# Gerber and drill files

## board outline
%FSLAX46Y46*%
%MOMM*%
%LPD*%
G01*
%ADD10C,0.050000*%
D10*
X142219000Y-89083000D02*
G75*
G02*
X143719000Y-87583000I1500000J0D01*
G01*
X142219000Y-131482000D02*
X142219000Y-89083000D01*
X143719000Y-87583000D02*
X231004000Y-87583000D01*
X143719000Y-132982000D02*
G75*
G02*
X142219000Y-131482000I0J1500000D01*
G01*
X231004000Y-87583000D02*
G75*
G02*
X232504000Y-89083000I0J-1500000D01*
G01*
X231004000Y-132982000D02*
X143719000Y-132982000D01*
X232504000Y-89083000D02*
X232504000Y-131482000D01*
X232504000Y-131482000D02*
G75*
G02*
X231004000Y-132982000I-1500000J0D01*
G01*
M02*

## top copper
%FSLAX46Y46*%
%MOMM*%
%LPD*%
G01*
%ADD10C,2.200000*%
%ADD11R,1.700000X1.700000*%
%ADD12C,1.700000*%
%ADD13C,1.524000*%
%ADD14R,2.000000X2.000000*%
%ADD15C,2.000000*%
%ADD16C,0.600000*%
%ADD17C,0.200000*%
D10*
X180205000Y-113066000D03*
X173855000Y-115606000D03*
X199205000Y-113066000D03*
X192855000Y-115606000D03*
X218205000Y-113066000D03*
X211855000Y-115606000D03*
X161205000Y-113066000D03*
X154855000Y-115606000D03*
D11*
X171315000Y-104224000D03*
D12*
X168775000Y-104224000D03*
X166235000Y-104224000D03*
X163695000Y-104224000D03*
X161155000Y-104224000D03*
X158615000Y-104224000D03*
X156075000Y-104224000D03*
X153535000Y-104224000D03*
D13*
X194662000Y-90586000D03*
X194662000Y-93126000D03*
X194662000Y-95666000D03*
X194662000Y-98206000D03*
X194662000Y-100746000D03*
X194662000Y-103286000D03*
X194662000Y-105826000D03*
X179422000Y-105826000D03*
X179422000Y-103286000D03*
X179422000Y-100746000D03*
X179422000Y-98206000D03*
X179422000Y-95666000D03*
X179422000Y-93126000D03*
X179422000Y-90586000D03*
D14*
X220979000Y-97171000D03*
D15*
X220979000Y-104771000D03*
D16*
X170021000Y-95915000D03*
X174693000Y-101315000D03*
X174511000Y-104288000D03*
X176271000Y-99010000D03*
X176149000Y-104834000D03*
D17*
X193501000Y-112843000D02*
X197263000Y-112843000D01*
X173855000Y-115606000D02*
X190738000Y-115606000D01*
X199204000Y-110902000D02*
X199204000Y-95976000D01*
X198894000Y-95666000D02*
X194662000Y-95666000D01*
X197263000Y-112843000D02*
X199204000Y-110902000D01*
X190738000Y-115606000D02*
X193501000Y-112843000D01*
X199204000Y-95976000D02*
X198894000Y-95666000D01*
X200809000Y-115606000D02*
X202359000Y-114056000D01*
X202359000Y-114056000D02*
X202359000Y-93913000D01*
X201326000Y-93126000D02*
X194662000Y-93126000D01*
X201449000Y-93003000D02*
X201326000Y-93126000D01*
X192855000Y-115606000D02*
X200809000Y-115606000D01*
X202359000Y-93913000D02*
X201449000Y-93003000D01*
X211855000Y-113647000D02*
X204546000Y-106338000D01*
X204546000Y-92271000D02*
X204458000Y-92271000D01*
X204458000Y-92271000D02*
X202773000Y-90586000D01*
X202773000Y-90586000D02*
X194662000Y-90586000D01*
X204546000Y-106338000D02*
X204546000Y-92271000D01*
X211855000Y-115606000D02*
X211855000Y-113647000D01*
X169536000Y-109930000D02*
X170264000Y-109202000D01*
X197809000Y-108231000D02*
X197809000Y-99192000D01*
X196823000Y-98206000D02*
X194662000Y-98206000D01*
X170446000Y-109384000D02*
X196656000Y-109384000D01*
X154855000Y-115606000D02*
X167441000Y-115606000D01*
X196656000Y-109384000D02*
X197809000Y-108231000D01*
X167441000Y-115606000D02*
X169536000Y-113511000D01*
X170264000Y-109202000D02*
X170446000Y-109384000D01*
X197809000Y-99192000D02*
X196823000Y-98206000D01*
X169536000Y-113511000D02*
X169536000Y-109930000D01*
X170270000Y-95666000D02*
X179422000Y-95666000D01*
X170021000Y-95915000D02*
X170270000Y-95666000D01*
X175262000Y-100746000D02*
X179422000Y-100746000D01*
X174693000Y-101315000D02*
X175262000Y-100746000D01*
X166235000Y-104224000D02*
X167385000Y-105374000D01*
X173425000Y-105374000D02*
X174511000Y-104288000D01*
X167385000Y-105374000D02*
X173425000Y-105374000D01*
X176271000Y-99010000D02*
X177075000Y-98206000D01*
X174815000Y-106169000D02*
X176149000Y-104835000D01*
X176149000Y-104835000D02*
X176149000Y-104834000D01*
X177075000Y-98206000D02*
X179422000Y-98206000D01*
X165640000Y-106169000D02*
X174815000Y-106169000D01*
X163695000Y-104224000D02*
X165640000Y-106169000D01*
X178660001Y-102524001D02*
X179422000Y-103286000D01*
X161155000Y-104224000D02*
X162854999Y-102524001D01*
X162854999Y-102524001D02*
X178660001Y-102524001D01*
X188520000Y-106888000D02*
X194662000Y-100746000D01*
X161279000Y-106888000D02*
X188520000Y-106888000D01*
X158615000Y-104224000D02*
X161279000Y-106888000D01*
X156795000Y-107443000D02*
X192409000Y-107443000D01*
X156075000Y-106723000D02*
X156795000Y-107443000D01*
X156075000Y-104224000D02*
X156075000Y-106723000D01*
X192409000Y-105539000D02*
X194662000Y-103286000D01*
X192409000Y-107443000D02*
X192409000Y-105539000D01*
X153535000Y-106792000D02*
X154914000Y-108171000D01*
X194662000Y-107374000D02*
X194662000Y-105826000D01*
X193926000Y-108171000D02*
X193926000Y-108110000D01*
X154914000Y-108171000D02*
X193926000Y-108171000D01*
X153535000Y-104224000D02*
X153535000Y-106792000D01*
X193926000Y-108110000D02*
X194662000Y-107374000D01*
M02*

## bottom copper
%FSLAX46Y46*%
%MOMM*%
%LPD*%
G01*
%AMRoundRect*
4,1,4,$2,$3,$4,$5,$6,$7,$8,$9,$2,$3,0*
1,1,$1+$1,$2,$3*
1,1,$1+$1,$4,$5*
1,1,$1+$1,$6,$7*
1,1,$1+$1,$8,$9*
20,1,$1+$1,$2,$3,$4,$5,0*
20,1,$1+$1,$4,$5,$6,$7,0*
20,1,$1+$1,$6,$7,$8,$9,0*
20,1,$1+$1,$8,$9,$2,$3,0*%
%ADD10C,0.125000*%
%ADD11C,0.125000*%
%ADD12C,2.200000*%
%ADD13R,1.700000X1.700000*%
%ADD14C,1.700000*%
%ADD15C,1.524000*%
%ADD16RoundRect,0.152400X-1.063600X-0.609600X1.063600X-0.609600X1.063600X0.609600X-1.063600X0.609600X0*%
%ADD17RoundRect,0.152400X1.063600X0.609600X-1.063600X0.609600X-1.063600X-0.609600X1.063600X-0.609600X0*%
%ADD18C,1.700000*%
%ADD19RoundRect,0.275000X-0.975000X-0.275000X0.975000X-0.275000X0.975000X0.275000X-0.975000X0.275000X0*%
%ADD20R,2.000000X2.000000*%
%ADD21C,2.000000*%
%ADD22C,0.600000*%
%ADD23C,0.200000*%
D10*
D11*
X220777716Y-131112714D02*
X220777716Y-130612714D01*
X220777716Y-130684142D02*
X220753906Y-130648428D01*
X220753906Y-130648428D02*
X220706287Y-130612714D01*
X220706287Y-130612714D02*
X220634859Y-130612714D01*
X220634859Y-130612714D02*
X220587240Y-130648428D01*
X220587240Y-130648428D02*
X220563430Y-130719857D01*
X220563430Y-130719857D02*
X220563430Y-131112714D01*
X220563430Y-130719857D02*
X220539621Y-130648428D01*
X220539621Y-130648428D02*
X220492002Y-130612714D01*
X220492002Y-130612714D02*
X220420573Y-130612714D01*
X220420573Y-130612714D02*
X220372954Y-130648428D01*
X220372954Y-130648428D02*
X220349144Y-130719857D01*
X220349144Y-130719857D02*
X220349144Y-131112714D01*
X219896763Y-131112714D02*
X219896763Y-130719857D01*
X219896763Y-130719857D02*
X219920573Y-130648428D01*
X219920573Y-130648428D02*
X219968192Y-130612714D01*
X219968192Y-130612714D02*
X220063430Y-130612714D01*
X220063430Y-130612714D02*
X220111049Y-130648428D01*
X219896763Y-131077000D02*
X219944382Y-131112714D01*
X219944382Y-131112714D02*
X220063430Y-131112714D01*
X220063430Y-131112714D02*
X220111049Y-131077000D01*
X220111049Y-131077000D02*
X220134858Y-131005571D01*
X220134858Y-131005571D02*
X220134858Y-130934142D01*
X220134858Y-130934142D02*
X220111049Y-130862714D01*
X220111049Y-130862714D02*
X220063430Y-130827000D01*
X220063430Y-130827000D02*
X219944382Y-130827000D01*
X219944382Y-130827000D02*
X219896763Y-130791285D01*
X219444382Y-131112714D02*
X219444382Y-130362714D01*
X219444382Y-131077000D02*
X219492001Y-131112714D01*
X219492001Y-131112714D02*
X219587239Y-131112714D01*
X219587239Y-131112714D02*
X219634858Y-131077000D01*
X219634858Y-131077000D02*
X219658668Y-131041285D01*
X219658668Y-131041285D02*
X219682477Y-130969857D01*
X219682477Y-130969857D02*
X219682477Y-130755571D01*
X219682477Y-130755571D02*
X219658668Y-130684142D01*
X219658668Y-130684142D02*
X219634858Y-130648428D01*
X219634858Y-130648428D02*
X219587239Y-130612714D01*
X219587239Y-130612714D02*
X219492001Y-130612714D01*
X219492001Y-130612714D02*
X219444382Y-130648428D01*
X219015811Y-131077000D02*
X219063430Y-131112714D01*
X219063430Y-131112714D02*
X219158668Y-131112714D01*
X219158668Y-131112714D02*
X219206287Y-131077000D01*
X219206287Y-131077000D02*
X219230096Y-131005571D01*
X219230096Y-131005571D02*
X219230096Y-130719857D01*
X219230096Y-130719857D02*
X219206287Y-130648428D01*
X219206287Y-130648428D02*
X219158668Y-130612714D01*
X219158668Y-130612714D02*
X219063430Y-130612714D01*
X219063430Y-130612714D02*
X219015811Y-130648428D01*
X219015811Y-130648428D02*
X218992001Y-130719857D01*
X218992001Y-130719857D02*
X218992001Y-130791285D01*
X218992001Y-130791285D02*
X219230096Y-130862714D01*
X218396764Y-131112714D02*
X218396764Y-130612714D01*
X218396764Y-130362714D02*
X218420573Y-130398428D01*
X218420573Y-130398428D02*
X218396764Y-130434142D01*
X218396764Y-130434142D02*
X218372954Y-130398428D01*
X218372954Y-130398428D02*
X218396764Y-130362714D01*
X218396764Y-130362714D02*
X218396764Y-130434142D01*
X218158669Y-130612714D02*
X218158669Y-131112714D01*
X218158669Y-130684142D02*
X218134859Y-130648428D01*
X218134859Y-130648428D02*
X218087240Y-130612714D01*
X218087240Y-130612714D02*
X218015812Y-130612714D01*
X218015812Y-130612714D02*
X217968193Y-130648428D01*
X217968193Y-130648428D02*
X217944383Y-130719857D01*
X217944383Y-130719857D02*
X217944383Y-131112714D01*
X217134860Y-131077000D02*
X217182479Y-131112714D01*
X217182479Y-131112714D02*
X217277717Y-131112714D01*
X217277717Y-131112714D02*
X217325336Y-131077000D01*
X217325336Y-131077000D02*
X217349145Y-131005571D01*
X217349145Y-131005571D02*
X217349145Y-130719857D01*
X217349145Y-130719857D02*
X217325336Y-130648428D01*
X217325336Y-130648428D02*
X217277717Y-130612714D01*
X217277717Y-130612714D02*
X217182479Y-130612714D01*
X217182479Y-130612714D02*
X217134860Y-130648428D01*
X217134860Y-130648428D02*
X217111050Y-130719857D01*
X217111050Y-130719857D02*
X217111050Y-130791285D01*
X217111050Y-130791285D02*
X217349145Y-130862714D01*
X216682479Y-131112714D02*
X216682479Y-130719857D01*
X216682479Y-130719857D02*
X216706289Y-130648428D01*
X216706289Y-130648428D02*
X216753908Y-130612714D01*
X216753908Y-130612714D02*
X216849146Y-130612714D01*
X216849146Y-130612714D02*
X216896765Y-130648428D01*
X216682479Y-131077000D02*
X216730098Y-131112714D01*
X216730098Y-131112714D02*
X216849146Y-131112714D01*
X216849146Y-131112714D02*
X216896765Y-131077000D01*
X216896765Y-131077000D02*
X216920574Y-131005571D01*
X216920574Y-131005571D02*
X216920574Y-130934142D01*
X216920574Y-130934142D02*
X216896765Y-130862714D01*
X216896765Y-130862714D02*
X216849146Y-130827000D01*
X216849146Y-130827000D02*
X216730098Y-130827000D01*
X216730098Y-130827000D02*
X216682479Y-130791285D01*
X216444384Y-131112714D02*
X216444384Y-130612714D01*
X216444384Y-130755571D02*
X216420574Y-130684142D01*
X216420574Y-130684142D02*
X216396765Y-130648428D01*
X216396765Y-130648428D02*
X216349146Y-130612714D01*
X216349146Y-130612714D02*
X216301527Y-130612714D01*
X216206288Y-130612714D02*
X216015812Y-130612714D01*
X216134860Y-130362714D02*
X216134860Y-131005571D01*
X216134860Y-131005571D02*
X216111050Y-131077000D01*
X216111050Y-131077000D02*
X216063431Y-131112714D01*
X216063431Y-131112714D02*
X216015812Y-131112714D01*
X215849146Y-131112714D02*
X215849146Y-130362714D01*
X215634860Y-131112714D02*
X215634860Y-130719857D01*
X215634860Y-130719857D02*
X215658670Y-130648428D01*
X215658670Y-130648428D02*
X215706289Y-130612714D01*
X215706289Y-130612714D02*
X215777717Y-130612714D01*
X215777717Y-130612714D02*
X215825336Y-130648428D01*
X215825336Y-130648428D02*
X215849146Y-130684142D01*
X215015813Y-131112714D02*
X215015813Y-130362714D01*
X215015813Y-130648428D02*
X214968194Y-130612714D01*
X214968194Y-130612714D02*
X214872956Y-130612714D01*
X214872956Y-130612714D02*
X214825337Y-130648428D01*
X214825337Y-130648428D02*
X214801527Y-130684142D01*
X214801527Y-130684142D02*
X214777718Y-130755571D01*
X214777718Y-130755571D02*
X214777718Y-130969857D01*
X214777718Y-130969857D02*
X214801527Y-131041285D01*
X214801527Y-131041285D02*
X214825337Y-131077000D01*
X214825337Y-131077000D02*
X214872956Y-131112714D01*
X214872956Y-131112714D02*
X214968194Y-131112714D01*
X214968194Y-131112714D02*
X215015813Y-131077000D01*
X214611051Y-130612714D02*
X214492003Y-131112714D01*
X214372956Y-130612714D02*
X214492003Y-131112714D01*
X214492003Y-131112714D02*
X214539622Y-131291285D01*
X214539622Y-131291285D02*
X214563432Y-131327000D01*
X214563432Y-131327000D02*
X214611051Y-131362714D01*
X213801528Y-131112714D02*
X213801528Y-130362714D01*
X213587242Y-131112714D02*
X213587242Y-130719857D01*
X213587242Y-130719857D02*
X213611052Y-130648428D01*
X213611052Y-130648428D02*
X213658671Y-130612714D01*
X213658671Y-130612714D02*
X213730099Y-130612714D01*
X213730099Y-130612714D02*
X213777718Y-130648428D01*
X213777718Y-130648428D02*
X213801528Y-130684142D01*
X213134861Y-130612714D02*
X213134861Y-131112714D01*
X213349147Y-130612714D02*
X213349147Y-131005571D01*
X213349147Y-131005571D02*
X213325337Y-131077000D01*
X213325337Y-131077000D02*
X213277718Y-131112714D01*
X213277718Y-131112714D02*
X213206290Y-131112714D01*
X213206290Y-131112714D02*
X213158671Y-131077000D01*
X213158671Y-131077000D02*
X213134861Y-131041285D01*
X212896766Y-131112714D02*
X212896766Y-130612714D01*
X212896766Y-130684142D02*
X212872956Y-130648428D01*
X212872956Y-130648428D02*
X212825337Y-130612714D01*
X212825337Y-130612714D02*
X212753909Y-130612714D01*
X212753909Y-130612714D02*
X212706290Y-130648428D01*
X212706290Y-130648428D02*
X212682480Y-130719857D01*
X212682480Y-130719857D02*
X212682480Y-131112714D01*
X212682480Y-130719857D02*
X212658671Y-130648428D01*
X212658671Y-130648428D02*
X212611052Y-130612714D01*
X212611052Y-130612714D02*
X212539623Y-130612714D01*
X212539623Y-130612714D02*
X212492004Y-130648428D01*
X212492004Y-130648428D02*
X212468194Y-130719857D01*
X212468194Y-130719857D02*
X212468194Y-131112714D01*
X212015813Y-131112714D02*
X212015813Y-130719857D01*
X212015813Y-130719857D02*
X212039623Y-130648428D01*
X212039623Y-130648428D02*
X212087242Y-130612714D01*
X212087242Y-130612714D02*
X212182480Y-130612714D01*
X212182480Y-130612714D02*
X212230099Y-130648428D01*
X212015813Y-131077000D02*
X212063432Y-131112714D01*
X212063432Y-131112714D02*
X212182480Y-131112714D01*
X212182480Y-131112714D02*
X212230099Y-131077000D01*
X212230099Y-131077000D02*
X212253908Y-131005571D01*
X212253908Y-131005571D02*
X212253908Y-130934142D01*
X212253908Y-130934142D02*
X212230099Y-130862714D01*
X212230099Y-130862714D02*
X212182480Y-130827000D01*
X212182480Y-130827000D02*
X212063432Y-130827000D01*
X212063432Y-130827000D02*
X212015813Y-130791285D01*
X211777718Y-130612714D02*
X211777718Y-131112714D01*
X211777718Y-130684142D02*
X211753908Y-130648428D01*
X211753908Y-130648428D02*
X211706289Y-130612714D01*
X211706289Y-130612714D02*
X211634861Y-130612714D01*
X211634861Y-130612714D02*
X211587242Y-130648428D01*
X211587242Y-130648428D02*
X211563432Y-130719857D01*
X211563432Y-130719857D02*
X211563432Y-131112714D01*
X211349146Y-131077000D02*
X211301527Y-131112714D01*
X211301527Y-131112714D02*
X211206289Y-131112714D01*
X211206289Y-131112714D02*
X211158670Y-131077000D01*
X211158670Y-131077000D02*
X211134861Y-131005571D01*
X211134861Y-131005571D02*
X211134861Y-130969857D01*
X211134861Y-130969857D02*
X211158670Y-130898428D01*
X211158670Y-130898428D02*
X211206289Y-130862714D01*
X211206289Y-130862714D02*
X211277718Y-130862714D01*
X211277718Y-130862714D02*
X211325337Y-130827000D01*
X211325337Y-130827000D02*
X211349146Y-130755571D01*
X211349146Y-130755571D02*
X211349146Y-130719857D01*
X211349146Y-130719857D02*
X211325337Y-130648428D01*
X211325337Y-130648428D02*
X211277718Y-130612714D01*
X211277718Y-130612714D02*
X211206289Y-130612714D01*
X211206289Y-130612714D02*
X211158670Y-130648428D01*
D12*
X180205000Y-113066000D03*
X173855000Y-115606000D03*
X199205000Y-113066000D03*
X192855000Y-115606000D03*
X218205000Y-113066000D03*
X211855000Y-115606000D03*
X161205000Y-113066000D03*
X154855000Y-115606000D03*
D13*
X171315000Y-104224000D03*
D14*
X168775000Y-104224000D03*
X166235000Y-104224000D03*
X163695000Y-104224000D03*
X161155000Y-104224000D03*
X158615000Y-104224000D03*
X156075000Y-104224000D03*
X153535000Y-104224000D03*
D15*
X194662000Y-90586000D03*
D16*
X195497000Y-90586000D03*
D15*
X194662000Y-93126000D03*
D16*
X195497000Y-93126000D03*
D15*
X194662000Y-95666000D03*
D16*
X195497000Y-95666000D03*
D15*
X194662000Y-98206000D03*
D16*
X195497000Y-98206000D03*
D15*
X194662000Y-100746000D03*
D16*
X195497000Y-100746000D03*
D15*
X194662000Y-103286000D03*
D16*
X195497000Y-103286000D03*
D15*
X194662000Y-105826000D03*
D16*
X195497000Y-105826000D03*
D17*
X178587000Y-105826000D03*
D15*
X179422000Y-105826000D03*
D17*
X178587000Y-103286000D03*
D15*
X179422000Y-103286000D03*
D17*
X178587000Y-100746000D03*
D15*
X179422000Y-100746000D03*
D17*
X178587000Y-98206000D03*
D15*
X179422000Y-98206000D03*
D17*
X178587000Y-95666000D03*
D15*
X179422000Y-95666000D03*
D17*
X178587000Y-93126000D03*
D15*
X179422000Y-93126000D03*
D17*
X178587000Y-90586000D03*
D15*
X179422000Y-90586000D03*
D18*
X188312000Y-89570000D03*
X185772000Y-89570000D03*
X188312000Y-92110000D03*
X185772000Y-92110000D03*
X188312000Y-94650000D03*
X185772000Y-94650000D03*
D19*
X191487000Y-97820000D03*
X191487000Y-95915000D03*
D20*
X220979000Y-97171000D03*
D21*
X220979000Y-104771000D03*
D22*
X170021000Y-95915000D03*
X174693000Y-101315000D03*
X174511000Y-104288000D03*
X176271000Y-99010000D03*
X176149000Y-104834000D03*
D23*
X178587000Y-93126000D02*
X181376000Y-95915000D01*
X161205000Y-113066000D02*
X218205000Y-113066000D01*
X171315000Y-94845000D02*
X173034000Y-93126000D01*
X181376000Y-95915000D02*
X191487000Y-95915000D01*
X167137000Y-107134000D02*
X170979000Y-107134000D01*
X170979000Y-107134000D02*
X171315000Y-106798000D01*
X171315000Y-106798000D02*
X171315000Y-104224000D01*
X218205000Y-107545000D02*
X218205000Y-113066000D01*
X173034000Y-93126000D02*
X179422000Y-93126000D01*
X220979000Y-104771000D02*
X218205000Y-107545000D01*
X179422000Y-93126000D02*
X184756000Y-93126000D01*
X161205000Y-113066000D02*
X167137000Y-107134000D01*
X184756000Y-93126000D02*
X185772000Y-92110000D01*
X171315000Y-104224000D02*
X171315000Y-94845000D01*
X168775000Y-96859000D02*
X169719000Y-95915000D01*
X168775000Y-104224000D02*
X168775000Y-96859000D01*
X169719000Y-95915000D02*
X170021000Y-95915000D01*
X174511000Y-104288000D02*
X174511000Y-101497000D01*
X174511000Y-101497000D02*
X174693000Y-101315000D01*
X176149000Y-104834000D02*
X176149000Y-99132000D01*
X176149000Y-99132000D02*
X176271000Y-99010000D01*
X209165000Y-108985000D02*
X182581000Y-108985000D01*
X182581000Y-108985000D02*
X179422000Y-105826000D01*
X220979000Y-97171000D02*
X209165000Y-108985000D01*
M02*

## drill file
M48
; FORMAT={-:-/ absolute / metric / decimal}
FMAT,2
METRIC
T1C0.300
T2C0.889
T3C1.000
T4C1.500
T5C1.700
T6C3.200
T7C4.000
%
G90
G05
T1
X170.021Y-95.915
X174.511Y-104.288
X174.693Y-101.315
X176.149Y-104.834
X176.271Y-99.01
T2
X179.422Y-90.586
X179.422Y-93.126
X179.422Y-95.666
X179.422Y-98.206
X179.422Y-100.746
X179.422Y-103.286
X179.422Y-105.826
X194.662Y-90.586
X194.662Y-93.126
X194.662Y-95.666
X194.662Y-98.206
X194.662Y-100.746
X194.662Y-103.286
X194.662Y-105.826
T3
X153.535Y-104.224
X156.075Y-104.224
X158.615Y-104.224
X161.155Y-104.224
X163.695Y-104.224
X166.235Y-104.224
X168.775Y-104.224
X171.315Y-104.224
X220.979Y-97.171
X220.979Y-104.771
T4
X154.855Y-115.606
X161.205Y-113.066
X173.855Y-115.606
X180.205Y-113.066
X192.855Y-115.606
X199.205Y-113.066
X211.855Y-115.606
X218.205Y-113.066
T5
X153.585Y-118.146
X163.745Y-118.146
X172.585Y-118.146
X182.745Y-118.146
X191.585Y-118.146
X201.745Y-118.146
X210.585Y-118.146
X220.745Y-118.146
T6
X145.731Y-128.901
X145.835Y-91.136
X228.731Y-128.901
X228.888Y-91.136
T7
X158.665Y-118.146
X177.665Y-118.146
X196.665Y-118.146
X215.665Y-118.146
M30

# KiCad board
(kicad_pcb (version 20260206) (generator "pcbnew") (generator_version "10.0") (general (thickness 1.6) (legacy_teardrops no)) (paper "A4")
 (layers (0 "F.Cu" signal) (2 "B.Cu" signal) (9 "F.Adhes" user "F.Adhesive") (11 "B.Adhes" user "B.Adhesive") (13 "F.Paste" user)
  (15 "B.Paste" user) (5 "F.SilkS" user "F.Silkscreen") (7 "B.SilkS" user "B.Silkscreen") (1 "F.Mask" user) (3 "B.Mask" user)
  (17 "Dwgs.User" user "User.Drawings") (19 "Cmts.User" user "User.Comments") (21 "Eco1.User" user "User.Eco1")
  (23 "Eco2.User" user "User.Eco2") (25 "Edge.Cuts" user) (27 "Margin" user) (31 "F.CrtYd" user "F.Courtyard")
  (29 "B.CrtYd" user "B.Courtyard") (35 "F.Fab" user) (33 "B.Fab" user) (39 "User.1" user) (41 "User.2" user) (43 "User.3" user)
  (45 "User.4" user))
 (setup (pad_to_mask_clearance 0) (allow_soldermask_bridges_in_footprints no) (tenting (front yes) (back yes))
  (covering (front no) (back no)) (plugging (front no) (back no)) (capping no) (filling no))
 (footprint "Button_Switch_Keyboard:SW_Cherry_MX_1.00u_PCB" (layer "F.Cu") (at 180.205 113.066)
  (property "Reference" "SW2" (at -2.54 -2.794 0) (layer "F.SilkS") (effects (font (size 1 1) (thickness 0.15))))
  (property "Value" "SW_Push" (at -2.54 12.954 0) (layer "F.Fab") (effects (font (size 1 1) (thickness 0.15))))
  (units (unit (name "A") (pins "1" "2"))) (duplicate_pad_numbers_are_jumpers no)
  (pad "" np_thru_hole circle (at -7.62 5.08) (size 1.7 1.7) (drill 1.7) (layers "*.Cu" "*.Mask"))
  (pad "" np_thru_hole circle (at -2.54 5.08) (size 4 4) (drill 4) (layers "*.Cu" "*.Mask"))
  (pad "" np_thru_hole circle (at 2.54 5.08) (size 1.7 1.7) (drill 1.7) (layers "*.Cu" "*.Mask"))
  (pad "1" thru_hole circle (at 0 0) (size 2.2 2.2) (drill 1.5) (layers "*.Cu" "*.Mask") (remove_unused_layers no) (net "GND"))
  (pad "2" thru_hole circle (at -6.35 2.54) (size 2.2 2.2) (drill 1.5) (layers "*.Cu" "*.Mask") (remove_unused_layers no)
   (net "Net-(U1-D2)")))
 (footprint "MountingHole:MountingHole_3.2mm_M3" (layer "F.Cu") (at 228.888 91.136)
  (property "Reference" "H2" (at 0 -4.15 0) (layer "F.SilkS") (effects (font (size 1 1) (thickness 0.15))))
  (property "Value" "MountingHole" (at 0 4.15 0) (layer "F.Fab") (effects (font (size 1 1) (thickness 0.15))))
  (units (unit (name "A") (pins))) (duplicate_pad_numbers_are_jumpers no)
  (pad "" np_thru_hole circle (at 0 0) (size 3.2 3.2) (drill 3.2) (layers "*.Cu" "*.Mask")))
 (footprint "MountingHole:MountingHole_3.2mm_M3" (layer "F.Cu") (at 145.731 128.901)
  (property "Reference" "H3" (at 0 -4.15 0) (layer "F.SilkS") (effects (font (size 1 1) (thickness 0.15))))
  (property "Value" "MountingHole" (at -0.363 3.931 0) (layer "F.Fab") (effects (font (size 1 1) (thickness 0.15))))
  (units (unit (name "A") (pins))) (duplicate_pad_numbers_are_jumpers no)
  (pad "" np_thru_hole circle (at 0 0) (size 3.2 3.2) (drill 3.2) (layers "*.Cu" "*.Mask")))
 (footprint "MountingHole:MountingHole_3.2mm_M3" (layer "F.Cu") (at 228.731 128.901)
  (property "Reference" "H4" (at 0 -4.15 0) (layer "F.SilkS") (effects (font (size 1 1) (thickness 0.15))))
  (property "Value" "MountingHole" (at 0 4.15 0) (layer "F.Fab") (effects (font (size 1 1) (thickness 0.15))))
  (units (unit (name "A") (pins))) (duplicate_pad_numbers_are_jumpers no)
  (pad "" np_thru_hole circle (at 0 0) (size 3.2 3.2) (drill 3.2) (layers "*.Cu" "*.Mask")))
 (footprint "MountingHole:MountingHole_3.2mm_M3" (layer "F.Cu") (at 145.835 91.136)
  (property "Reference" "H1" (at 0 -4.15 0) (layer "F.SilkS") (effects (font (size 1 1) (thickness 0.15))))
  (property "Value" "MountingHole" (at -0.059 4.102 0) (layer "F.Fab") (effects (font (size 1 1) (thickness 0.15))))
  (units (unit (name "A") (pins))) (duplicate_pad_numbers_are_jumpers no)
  (pad "" np_thru_hole circle (at 0 0) (size 3.2 3.2) (drill 3.2) (layers "*.Cu" "*.Mask")))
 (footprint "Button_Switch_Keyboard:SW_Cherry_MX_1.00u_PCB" (layer "F.Cu") (at 199.205 113.066)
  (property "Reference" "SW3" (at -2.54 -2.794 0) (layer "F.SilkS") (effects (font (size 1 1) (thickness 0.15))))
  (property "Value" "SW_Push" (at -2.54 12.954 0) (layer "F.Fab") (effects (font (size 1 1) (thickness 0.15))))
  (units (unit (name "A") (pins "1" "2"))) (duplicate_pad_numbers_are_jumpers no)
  (pad "" np_thru_hole circle (at -7.62 5.08) (size 1.7 1.7) (drill 1.7) (layers "*.Cu" "*.Mask"))
  (pad "" np_thru_hole circle (at -2.54 5.08) (size 4 4) (drill 4) (layers "*.Cu" "*.Mask"))
  (pad "" np_thru_hole circle (at 2.54 5.08) (size 1.7 1.7) (drill 1.7) (layers "*.Cu" "*.Mask"))
  (pad "1" thru_hole circle (at 0 0) (size 2.2 2.2) (drill 1.5) (layers "*.Cu" "*.Mask") (remove_unused_layers no) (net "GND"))
  (pad "2" thru_hole circle (at -6.35 2.54) (size 2.2 2.2) (drill 1.5) (layers "*.Cu" "*.Mask") (remove_unused_layers no)
   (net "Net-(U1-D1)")))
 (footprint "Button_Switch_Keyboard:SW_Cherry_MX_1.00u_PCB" (layer "F.Cu") (at 218.205 113.066)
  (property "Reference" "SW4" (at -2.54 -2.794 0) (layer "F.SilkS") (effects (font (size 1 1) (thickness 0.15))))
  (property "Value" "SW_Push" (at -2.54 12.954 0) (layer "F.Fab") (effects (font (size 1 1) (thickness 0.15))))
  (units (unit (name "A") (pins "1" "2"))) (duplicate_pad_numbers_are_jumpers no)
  (pad "" np_thru_hole circle (at -7.62 5.08) (size 1.7 1.7) (drill 1.7) (layers "*.Cu" "*.Mask"))
  (pad "" np_thru_hole circle (at -2.54 5.08) (size 4 4) (drill 4) (layers "*.Cu" "*.Mask"))
  (pad "" np_thru_hole circle (at 2.54 5.08) (size 1.7 1.7) (drill 1.7) (layers "*.Cu" "*.Mask"))
  (pad "1" thru_hole circle (at 0 0) (size 2.2 2.2) (drill 1.5) (layers "*.Cu" "*.Mask") (remove_unused_layers no) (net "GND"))
  (pad "2" thru_hole circle (at -6.35 2.54) (size 2.2 2.2) (drill 1.5) (layers "*.Cu" "*.Mask") (remove_unused_layers no)
   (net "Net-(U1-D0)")))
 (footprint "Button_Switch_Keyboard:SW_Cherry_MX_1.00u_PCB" (layer "F.Cu") (at 161.205 113.066)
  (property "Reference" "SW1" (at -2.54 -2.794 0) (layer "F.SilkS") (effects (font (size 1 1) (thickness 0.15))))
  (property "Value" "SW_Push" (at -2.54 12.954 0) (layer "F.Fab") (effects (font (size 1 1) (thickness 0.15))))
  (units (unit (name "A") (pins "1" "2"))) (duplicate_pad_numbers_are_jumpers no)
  (pad "" np_thru_hole circle (at -7.62 5.08) (size 1.7 1.7) (drill 1.7) (layers "*.Cu" "*.Mask"))
  (pad "" np_thru_hole circle (at -2.54 5.08) (size 4 4) (drill 4) (layers "*.Cu" "*.Mask"))
  (pad "" np_thru_hole circle (at 2.54 5.08) (size 1.7 1.7) (drill 1.7) (layers "*.Cu" "*.Mask"))
  (pad "1" thru_hole circle (at 0 0) (size 2.2 2.2) (drill 1.5) (layers "*.Cu" "*.Mask") (remove_unused_layers no) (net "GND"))
  (pad "2" thru_hole circle (at -6.35 2.54) (size 2.2 2.2) (drill 1.5) (layers "*.Cu" "*.Mask") (remove_unused_layers no)
   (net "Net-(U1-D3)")))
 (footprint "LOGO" (layer "F.Cu") (at 158.714 92.166)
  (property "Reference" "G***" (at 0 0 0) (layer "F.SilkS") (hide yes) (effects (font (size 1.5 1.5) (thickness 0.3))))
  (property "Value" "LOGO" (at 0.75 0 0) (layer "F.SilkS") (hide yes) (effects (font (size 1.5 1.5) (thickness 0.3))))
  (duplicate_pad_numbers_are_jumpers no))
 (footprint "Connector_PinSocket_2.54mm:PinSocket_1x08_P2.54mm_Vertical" (layer "B.Cu") (at 171.315 104.224 90)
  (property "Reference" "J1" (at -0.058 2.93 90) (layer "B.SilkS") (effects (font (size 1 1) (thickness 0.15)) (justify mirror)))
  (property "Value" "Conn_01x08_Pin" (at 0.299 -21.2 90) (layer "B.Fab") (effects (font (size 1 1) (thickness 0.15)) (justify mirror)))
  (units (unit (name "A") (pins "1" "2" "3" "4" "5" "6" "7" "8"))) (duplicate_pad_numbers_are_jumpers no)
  (pad "1" thru_hole rect (at 0 0 90) (size 1.7 1.7) (drill 1) (layers "*.Cu" "*.Mask") (remove_unused_layers no) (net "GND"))
  (pad "2" thru_hole circle (at 0 -2.54 90) (size 1.7 1.7) (drill 1) (layers "*.Cu" "*.Mask") (remove_unused_layers no) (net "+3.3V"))
  (pad "3" thru_hole circle (at 0 -5.08 90) (size 1.7 1.7) (drill 1) (layers "*.Cu" "*.Mask") (remove_unused_layers no) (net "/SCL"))
  (pad "4" thru_hole circle (at 0 -7.62 90) (size 1.7 1.7) (drill 1) (layers "*.Cu" "*.Mask") (remove_unused_layers no) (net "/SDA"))
  (pad "5" thru_hole circle (at 0 -10.16 90) (size 1.7 1.7) (drill 1) (layers "*.Cu" "*.Mask") (remove_unused_layers no) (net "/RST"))
  (pad "6" thru_hole circle (at 0 -12.7 90) (size 1.7 1.7) (drill 1) (layers "*.Cu" "*.Mask") (remove_unused_layers no) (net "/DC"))
  (pad "7" thru_hole circle (at 0 -15.24 90) (size 1.7 1.7) (drill 1) (layers "*.Cu" "*.Mask") (remove_unused_layers no) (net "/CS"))
  (pad "8" thru_hole circle (at 0 -17.78 90) (size 1.7 1.7) (drill 1) (layers "*.Cu" "*.Mask") (remove_unused_layers no) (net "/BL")))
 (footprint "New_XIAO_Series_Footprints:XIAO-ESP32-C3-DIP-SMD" (layer "B.Cu") (at 187.042 98.206 90)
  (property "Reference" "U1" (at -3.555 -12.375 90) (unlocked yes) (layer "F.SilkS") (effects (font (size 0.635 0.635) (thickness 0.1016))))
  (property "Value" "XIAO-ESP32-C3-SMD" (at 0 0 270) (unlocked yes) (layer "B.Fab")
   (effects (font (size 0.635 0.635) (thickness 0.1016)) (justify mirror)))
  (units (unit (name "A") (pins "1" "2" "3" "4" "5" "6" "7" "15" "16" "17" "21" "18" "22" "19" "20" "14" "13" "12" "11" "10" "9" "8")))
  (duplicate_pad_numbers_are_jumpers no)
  (pad "1" thru_hole circle (at 7.62 7.62) (size 1.524 1.524) (drill 0.889) (layers "*.Cu" "*.Mask") (remove_unused_layers no)
   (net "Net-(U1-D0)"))
  (pad "1" smd roundrect (at 7.62 8.455) (size 2.432 1.524) (layers "B.Cu" "B.Mask") (roundrect_rratio 0.1) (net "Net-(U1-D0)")
   (thermal_bridge_angle 45))
  (pad "2" thru_hole circle (at 5.08 7.62) (size 1.524 1.524) (drill 0.889) (layers "*.Cu" "*.Mask") (remove_unused_layers no)
   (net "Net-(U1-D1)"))
  (pad "2" smd roundrect (at 5.08 8.455) (size 2.432 1.524) (layers "B.Cu" "B.Mask") (roundrect_rratio 0.1) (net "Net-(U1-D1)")
   (thermal_bridge_angle 45))
  (pad "3" thru_hole circle (at 2.54 7.62) (size 1.524 1.524) (drill 0.889) (layers "*.Cu" "*.Mask") (remove_unused_layers no)
   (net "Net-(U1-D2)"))
  (pad "3" smd roundrect (at 2.54 8.455) (size 2.432 1.524) (layers "B.Cu" "B.Mask") (roundrect_rratio 0.1) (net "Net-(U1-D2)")
   (thermal_bridge_angle 45))
  (pad "4" thru_hole circle (at 0 7.62) (size 1.524 1.524) (drill 0.889) (layers "*.Cu" "*.Mask") (remove_unused_layers no)
   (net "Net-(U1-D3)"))
  (pad "4" smd roundrect (at 0 8.455) (size 2.432 1.524) (layers "B.Cu" "B.Mask") (roundrect_rratio 0.1) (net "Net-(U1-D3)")
   (thermal_bridge_angle 45))
  (pad "5" thru_hole circle (at -2.54 7.62) (size 1.524 1.524) (drill 0.889) (layers "*.Cu" "*.Mask") (remove_unused_layers no) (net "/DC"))
  (pad "5" smd roundrect (at -2.54 8.455) (size 2.432 1.524) (layers "B.Cu" "B.Mask") (roundrect_rratio 0.1) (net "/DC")
   (thermal_bridge_angle 45))
  (pad "6" thru_hole circle (at -5.08 7.62) (size 1.524 1.524) (drill 0.889) (layers "*.Cu" "*.Mask") (remove_unused_layers no) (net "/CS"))
  (pad "6" smd roundrect (at -5.08 8.455) (size 2.432 1.524) (layers "B.Cu" "B.Mask") (roundrect_rratio 0.1) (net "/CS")
   (thermal_bridge_angle 45))
  (pad "7" thru_hole circle (at -7.62 7.62) (size 1.524 1.524) (drill 0.889) (layers "*.Cu" "*.Mask") (remove_unused_layers no) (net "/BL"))
  (pad "7" smd roundrect (at -7.62 8.455) (size 2.432 1.524) (layers "B.Cu" "B.Mask") (roundrect_rratio 0.1) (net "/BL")
   (thermal_bridge_angle 45))
  (pad "8" smd roundrect (at -7.62 -8.455 180) (size 2.432 1.524) (layers "B.Cu" "B.Mask") (roundrect_rratio 0.1) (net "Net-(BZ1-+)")
   (thermal_bridge_angle 45))
  (pad "8" thru_hole circle (at -7.62 -7.62 180) (size 1.524 1.524) (drill 0.889) (layers "*.Cu" "*.Mask") (remove_unused_layers no)
   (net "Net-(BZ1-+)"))
  (pad "9" smd roundrect (at -5.08 -8.455 180) (size 2.432 1.524) (layers "B.Cu" "B.Mask") (roundrect_rratio 0.1) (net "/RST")
   (thermal_bridge_angle 45))
  (pad "9" thru_hole circle (at -5.08 -7.62 180) (size 1.524 1.524) (drill 0.889) (layers "*.Cu" "*.Mask") (remove_unused_layers no)
   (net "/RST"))
  (pad "10" smd roundrect (at -2.54 -8.455 180) (size 2.432 1.524) (layers "B.Cu" "B.Mask") (roundrect_rratio 0.1) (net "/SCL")
   (thermal_bridge_angle 45))
  (pad "10" thru_hole circle (at -2.54 -7.62 180) (size 1.524 1.524) (drill 0.889) (layers "*.Cu" "*.Mask") (remove_unused_layers no)
   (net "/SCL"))
  (pad "11" smd roundrect (at 0 -8.455 180) (size 2.432 1.524) (layers "B.Cu" "B.Mask") (roundrect_rratio 0.1) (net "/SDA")
   (thermal_bridge_angle 45))
  (pad "11" thru_hole circle (at 0 -7.62 180) (size 1.524 1.524) (drill 0.889) (layers "*.Cu" "*.Mask") (remove_unused_layers no)
   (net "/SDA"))
  (pad "12" smd roundrect (at 2.54 -8.455 180) (size 2.432 1.524) (layers "B.Cu" "B.Mask") (roundrect_rratio 0.1) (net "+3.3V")
   (thermal_bridge_angle 45))
  (pad "12" thru_hole circle (at 2.54 -7.62 180) (size 1.524 1.524) (drill 0.889) (layers "*.Cu" "*.Mask") (remove_unused_layers no)
   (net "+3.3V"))
  (pad "13" smd roundrect (at 5.08 -8.455 180) (size 2.432 1.524) (layers "B.Cu" "B.Mask") (roundrect_rratio 0.1) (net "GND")
   (thermal_bridge_angle 45))
  (pad "13" thru_hole circle (at 5.08 -7.62 180) (size 1.524 1.524) (drill 0.889) (layers "*.Cu" "*.Mask") (remove_unused_layers no)
   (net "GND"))
  (pad "14" smd roundrect (at 7.62 -8.455 180) (size 2.432 1.524) (layers "B.Cu" "B.Mask") (roundrect_rratio 0.1)
   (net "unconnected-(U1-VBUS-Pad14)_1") (thermal_bridge_angle 45))
  (pad "14" thru_hole circle (at 7.62 -7.62 180) (size 1.524 1.524) (drill 0.889) (layers "*.Cu" "*.Mask") (remove_unused_layers no)
   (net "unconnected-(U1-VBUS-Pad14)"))
  (pad "15" smd circle (at 8.636 1.27 180) (size 1.7 1.7) (layers "B.Cu" "B.Mask" "B.Paste") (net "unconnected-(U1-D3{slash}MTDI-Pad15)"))
  (pad "16" smd circle (at 8.636 -1.27 180) (size 1.7 1.7) (layers "B.Cu" "B.Mask" "B.Paste") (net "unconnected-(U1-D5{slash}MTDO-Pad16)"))
  (pad "17" smd circle (at 6.096 1.27 180) (size 1.7 1.7) (layers "B.Cu" "B.Mask" "B.Paste") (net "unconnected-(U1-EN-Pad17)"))
  (pad "18" smd circle (at 6.096 -1.27 180) (size 1.7 1.7) (layers "B.Cu" "B.Mask" "B.Paste") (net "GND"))
  (pad "19" smd circle (at 3.556 1.27 180) (size 1.7 1.7) (layers "B.Cu" "B.Mask" "B.Paste") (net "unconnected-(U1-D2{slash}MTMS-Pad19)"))
  (pad "20" smd circle (at 3.556 -1.27 180) (size 1.7 1.7) (layers "B.Cu" "B.Mask" "B.Paste") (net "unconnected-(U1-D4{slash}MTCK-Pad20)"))
  (pad "21" smd roundrect (at 0.386 4.445) (size 2.5 1.1) (layers "B.Cu" "B.Mask" "B.Paste") (roundrect_rratio 0.25)
   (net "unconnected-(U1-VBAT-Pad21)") (thermal_bridge_angle 45))
  (pad "22" smd roundrect (at 2.291 4.445) (size 2.5 1.1) (layers "B.Cu" "B.Mask" "B.Paste") (roundrect_rratio 0.25) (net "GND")
   (thermal_bridge_angle 45)))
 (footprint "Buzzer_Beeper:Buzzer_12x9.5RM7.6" (layer "B.Cu") (at 220.979 97.171 -90)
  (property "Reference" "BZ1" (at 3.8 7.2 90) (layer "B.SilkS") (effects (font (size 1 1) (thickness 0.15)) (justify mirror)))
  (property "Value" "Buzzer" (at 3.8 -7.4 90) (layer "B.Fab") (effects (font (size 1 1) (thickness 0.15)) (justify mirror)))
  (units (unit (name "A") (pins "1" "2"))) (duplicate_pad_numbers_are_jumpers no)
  (pad "1" thru_hole rect (at 0 0 270) (size 2 2) (drill 1) (layers "*.Cu" "*.Mask") (remove_unused_layers no) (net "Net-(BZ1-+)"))
  (pad "2" thru_hole circle (at 7.6 0 270) (size 2 2) (drill 1) (layers "*.Cu" "*.Mask") (remove_unused_layers no) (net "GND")))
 (gr_arc (start 142.219 89.083) (mid 142.65834 88.02234) (end 143.719 87.583) (stroke (width 0.05) (type default)) (layer "Edge.Cuts"))
 (gr_line (start 142.219 131.482) (end 142.219 89.083) (stroke (width 0.05) (type default)) (layer "Edge.Cuts"))
 (gr_line (start 143.719 87.583) (end 231.004 87.583) (stroke (width 0.05) (type default)) (layer "Edge.Cuts"))
 (gr_arc (start 143.719 132.982) (mid 142.65834 132.54266) (end 142.219 131.482) (stroke (width 0.05) (type default)) (layer "Edge.Cuts"))
 (gr_arc (start 231.004 87.583) (mid 232.06466 88.02234) (end 232.504 89.083) (stroke (width 0.05) (type default)) (layer "Edge.Cuts"))
 (gr_line (start 231.004 132.982) (end 143.719 132.982) (stroke (width 0.05) (type default)) (layer "Edge.Cuts"))
 (gr_line (start 232.504 89.083) (end 232.504 131.482) (stroke (width 0.05) (type default)) (layer "Edge.Cuts"))
 (gr_arc (start 232.504 131.482) (mid 232.06466 132.54266) (end 231.004 132.982) (stroke (width 0.05) (type default)) (layer "Edge.Cuts"))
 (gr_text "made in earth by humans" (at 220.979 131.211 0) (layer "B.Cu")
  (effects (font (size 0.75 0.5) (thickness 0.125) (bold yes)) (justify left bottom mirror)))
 (segment (start 178.587 93.126) (end 181.376 95.915) (width 0.2) (layer "B.Cu") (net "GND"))
 (segment (start 161.205 113.066) (end 218.205 113.066) (width 0.2) (layer "B.Cu") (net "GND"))
 (segment (start 171.315 94.845) (end 173.034 93.126) (width 0.2) (layer "B.Cu") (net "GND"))
 (segment (start 181.376 95.915) (end 191.487 95.915) (width 0.2) (layer "B.Cu") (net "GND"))
 (segment (start 167.137 107.134) (end 170.979 107.134) (width 0.2) (layer "B.Cu") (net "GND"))
 (segment (start 170.979 107.134) (end 171.315 106.798) (width 0.2) (layer "B.Cu") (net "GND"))
 (segment (start 171.315 106.798) (end 171.315 104.224) (width 0.2) (layer "B.Cu") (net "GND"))
 (segment (start 218.205 107.545) (end 218.205 113.066) (width 0.2) (layer "B.Cu") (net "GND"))
 (segment (start 173.034 93.126) (end 179.422 93.126) (width 0.2) (layer "B.Cu") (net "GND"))
 (segment (start 220.979 104.771) (end 218.205 107.545) (width 0.2) (layer "B.Cu") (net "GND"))
 (segment (start 179.422 93.126) (end 184.756 93.126) (width 0.2) (layer "B.Cu") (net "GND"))
 (segment (start 161.205 113.066) (end 167.137 107.134) (width 0.2) (layer "B.Cu") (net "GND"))
 (segment (start 184.756 93.126) (end 185.772 92.11) (width 0.2) (layer "B.Cu") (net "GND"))
 (segment (start 171.315 104.224) (end 171.315 94.845) (width 0.2) (layer "B.Cu") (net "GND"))
 (segment (start 193.501 112.843) (end 197.263 112.843) (width 0.2) (layer "F.Cu") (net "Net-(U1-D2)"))
 (segment (start 173.855 115.606) (end 190.738 115.606) (width 0.2) (layer "F.Cu") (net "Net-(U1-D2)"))
 (segment (start 199.204 110.902) (end 199.204 95.976) (width 0.2) (layer "F.Cu") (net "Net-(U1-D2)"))
 (segment (start 198.894 95.666) (end 194.662 95.666) (width 0.2) (layer "F.Cu") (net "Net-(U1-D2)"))
 (segment (start 197.263 112.843) (end 199.204 110.902) (width 0.2) (layer "F.Cu") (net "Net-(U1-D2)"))
 (segment (start 190.738 115.606) (end 193.501 112.843) (width 0.2) (layer "F.Cu") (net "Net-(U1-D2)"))
 (segment (start 199.204 95.976) (end 198.894 95.666) (width 0.2) (layer "F.Cu") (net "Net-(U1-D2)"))
 (segment (start 200.809 115.606) (end 202.359 114.056) (width 0.2) (layer "F.Cu") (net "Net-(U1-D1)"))
 (segment (start 202.359 114.056) (end 202.359 93.913) (width 0.2) (layer "F.Cu") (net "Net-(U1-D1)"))
 (segment (start 201.326 93.126) (end 194.662 93.126) (width 0.2) (layer "F.Cu") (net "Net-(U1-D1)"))
 (segment (start 201.449 93.003) (end 201.326 93.126) (width 0.2) (layer "F.Cu") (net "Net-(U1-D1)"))
 (segment (start 192.855 115.606) (end 200.809 115.606) (width 0.2) (layer "F.Cu") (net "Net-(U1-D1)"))
 (segment (start 202.359 93.913) (end 201.449 93.003) (width 0.2) (layer "F.Cu") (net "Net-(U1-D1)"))
 (segment (start 211.855 113.647) (end 204.546 106.338) (width 0.2) (layer "F.Cu") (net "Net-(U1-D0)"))
 (segment (start 204.546 92.271) (end 204.458 92.271) (width 0.2) (layer "F.Cu") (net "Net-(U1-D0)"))
 (segment (start 204.458 92.271) (end 202.773 90.586) (width 0.2) (layer "F.Cu") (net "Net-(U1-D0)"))
 (segment (start 202.773 90.586) (end 194.662 90.586) (width 0.2) (layer "F.Cu") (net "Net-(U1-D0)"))
 (segment (start 204.546 106.338) (end 204.546 92.271) (width 0.2) (layer "F.Cu") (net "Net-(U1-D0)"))
 (segment (start 211.855 115.606) (end 211.855 113.647) (width 0.2) (layer "F.Cu") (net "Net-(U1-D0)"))
 (segment (start 169.536 109.93) (end 170.264 109.202) (width 0.2) (layer "F.Cu") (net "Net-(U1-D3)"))
 (segment (start 197.809 108.231) (end 197.809 99.192) (width 0.2) (layer "F.Cu") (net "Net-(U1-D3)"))
 (segment (start 196.823 98.206) (end 194.662 98.206) (width 0.2) (layer "F.Cu") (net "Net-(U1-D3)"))
 (segment (start 170.446 109.384) (end 196.656 109.384) (width 0.2) (layer "F.Cu") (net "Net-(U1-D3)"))
 (segment (start 154.855 115.606) (end 167.441 115.606) (width 0.2) (layer "F.Cu") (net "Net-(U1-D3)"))
 (segment (start 196.656 109.384) (end 197.809 108.231) (width 0.2) (layer "F.Cu") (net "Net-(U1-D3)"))
 (segment (start 167.441 115.606) (end 169.536 113.511) (width 0.2) (layer "F.Cu") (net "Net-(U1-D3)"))
 (segment (start 170.264 109.202) (end 170.446 109.384) (width 0.2) (layer "F.Cu") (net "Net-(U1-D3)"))
 (segment (start 197.809 99.192) (end 196.823 98.206) (width 0.2) (layer "F.Cu") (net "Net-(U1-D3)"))
 (segment (start 169.536 113.511) (end 169.536 109.93) (width 0.2) (layer "F.Cu") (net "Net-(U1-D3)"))
 (segment (start 170.27 95.666) (end 179.422 95.666) (width 0.2) (layer "F.Cu") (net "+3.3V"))
 (segment (start 170.021 95.915) (end 170.27 95.666) (width 0.2) (layer "F.Cu") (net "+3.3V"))
 (via (at 170.021 95.915) (size 0.6) (drill 0.3) (layers "F.Cu" "B.Cu") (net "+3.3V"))
 (segment (start 168.775 96.859) (end 169.719 95.915) (width 0.2) (layer "B.Cu") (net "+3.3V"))
 (segment (start 168.775 104.224) (end 168.775 96.859) (width 0.2) (layer "B.Cu") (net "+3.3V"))
 (segment (start 169.719 95.915) (end 170.021 95.915) (width 0.2) (layer "B.Cu") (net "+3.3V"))
 (segment (start 175.262 100.746) (end 179.422 100.746) (width 0.2) (layer "F.Cu") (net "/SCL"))
 (segment (start 174.693 101.315) (end 175.262 100.746) (width 0.2) (layer "F.Cu") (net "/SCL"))
 (segment (start 166.235 104.224) (end 167.385 105.374) (width 0.2) (layer "F.Cu") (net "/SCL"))
 (segment (start 173.425 105.374) (end 174.511 104.288) (width 0.2) (layer "F.Cu") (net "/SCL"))
 (segment (start 167.385 105.374) (end 173.425 105.374) (width 0.2) (layer "F.Cu") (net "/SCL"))
 (via (at 174.693 101.315) (size 0.6) (drill 0.3) (layers "F.Cu" "B.Cu") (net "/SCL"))
 (via (at 174.511 104.288) (size 0.6) (drill 0.3) (layers "F.Cu" "B.Cu") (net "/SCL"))
 (segment (start 174.511 104.288) (end 174.511 101.497) (width 0.2) (layer "B.Cu") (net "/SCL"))
 (segment (start 174.511 101.497) (end 174.693 101.315) (width 0.2) (layer "B.Cu") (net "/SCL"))
 (segment (start 176.271 99.01) (end 177.075 98.206) (width 0.2) (layer "F.Cu") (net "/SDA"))
 (segment (start 174.815 106.169) (end 176.149 104.835) (width 0.2) (layer "F.Cu") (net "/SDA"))
 (segment (start 176.149 104.835) (end 176.149 104.834) (width 0.2) (layer "F.Cu") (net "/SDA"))
 (segment (start 177.075 98.206) (end 179.422 98.206) (width 0.2) (layer "F.Cu") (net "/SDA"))
 (segment (start 165.64 106.169) (end 174.815 106.169) (width 0.2) (layer "F.Cu") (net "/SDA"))
 (segment (start 163.695 104.224) (end 165.64 106.169) (width 0.2) (layer "F.Cu") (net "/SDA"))
 (via (at 176.271 99.01) (size 0.6) (drill 0.3) (layers "F.Cu" "B.Cu") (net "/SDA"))
 (via (at 176.149 104.834) (size 0.6) (drill 0.3) (layers "F.Cu" "B.Cu") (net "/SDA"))
 (segment (start 176.149 104.834) (end 176.149 99.132) (width 0.2) (layer "B.Cu") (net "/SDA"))
 (segment (start 176.149 99.132) (end 176.271 99.01) (width 0.2) (layer "B.Cu") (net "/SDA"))
 (segment (start 178.660001 102.524001) (end 179.422 103.286) (width 0.2) (layer "F.Cu") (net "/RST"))
 (segment (start 161.155 104.224) (end 162.854999 102.524001) (width 0.2) (layer "F.Cu") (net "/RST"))
 (segment (start 162.854999 102.524001) (end 178.660001 102.524001) (width 0.2) (layer "F.Cu") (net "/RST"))
 (segment (start 188.52 106.888) (end 194.662 100.746) (width 0.2) (layer "F.Cu") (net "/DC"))
 (segment (start 161.279 106.888) (end 188.52 106.888) (width 0.2) (layer "F.Cu") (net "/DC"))
 (segment (start 158.615 104.224) (end 161.279 106.888) (width 0.2) (layer "F.Cu") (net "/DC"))
 (segment (start 156.795 107.443) (end 192.409 107.443) (width 0.2) (layer "F.Cu") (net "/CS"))
 (segment (start 156.075 106.723) (end 156.795 107.443) (width 0.2) (layer "F.Cu") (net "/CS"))
 (segment (start 156.075 104.224) (end 156.075 106.723) (width 0.2) (layer "F.Cu") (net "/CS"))
 (segment (start 192.409 105.539) (end 194.662 103.286) (width 0.2) (layer "F.Cu") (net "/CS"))
 (segment (start 192.409 107.443) (end 192.409 105.539) (width 0.2) (layer "F.Cu") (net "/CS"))
 (segment (start 153.535 106.792) (end 154.914 108.171) (width 0.2) (layer "F.Cu") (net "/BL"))
 (segment (start 194.662 107.374) (end 194.662 105.826) (width 0.2) (layer "F.Cu") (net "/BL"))
 (segment (start 193.926 108.171) (end 193.926 108.11) (width 0.2) (layer "F.Cu") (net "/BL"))
 (segment (start 154.914 108.171) (end 193.926 108.171) (width 0.2) (layer "F.Cu") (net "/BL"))
 (segment (start 153.535 104.224) (end 153.535 106.792) (width 0.2) (layer "F.Cu") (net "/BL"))
 (segment (start 193.926 108.11) (end 194.662 107.374) (width 0.2) (layer "F.Cu") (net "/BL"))
 (segment (start 209.165 108.985) (end 182.581 108.985) (width 0.2) (layer "B.Cu") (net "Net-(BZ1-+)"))
 (segment (start 182.581 108.985) (end 179.422 105.826) (width 0.2) (layer "B.Cu") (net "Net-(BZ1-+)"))
 (segment (start 220.979 97.171) (end 209.165 108.985) (width 0.2) (layer "B.Cu") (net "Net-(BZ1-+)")))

